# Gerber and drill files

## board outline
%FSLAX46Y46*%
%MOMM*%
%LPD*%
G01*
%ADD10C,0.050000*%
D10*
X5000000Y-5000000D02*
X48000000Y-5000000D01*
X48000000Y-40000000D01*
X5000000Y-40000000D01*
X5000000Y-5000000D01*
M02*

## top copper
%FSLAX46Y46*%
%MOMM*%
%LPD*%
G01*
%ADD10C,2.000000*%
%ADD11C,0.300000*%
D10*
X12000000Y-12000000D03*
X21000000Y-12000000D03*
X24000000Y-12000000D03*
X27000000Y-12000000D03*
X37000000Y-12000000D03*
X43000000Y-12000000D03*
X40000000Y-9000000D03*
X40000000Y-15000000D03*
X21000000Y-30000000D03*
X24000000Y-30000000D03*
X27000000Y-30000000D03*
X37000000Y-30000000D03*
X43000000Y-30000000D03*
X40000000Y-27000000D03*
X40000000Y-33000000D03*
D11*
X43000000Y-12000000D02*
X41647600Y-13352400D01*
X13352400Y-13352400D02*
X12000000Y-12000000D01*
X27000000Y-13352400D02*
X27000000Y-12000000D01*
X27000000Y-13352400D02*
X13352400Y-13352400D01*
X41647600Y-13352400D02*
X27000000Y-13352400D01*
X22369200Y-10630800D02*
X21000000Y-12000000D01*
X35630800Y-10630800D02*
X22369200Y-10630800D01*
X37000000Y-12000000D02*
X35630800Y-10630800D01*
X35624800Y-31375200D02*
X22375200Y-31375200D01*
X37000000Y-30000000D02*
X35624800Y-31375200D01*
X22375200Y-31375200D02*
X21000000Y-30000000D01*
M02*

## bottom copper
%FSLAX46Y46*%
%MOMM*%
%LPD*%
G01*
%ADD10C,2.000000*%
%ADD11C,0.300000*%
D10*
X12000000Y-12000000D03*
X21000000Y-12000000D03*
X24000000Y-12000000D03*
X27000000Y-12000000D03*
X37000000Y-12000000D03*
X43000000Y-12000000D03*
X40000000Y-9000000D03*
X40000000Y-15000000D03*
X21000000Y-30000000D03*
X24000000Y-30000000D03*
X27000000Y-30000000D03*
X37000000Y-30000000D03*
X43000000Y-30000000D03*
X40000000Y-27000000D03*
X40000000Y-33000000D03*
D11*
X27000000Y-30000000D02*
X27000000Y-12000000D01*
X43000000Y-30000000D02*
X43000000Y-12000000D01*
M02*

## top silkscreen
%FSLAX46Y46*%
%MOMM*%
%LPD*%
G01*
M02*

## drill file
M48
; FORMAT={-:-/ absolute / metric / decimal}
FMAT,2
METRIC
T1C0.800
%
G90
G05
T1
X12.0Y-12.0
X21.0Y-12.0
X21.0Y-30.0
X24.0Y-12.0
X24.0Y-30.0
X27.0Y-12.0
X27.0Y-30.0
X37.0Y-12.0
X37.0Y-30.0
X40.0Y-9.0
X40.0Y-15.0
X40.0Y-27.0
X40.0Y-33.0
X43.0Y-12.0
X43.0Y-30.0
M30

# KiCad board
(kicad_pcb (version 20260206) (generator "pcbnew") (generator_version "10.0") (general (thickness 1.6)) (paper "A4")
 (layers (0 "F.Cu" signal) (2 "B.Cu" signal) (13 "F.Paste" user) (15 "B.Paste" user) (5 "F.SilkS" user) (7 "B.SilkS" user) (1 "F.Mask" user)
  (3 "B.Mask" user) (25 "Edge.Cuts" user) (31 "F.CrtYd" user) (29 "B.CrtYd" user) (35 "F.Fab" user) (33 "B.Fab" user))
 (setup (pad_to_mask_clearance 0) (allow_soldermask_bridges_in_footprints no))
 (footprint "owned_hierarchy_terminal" (layer "F.Cu") (at 12 12)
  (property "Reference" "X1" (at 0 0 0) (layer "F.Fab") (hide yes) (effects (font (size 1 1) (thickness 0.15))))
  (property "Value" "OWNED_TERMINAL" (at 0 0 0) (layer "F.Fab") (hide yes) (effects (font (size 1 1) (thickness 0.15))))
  (pad "1" thru_hole circle (at 0 0) (size 2 2) (drill 0.8) (layers "*.Cu" "*.Mask") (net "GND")))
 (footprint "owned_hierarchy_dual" (layer "F.Cu") (at 24 12)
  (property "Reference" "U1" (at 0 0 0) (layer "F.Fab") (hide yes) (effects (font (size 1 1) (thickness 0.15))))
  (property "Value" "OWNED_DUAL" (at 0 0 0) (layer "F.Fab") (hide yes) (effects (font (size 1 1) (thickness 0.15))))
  (pad "1" thru_hole circle (at -3 0) (size 2 2) (drill 0.8) (layers "*.Cu" "*.Mask") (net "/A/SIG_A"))
  (pad "2" thru_hole circle (at 0 0) (size 2 2) (drill 0.8) (layers "*.Cu" "*.Mask") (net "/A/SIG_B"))
  (pad "3" thru_hole circle (at 3 0) (size 2 2) (drill 0.8) (layers "*.Cu" "*.Mask") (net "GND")))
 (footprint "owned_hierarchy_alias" (layer "F.Cu") (at 40 12)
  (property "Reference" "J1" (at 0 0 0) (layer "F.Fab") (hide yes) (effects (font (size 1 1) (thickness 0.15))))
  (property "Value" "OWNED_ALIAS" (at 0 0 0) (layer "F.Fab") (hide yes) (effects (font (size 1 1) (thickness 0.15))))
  (pad "R" thru_hole circle (at -3 0) (size 2 2) (drill 0.8) (layers "*.Cu" "*.Mask") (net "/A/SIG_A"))
  (pad "T" thru_hole circle (at 3 0) (size 2 2) (drill 0.8) (layers "*.Cu" "*.Mask") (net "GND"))
  (pad "MP" thru_hole circle (at 0 -3) (size 2 2) (drill 0.8) (layers "*.Cu" "*.Mask"))
  (pad "MP" thru_hole circle (at 0 3) (size 2 2) (drill 0.8) (layers "*.Cu" "*.Mask")))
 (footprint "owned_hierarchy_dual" (layer "F.Cu") (at 24 30)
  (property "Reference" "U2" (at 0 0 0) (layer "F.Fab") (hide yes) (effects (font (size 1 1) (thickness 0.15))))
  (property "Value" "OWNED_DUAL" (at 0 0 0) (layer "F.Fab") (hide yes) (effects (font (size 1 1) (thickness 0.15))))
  (pad "1" thru_hole circle (at -3 0) (size 2 2) (drill 0.8) (layers "*.Cu" "*.Mask") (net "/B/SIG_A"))
  (pad "2" thru_hole circle (at 0 0) (size 2 2) (drill 0.8) (layers "*.Cu" "*.Mask") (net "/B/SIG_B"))
  (pad "3" thru_hole circle (at 3 0) (size 2 2) (drill 0.8) (layers "*.Cu" "*.Mask") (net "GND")))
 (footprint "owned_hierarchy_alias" (layer "F.Cu") (at 40 30)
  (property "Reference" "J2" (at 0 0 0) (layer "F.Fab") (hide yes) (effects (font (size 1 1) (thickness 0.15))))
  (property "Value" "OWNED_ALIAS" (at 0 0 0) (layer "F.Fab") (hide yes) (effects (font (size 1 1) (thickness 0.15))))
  (pad "R" thru_hole circle (at -3 0) (size 2 2) (drill 0.8) (layers "*.Cu" "*.Mask") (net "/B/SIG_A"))
  (pad "T" thru_hole circle (at 3 0) (size 2 2) (drill 0.8) (layers "*.Cu" "*.Mask") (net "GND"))
  (pad "MP" thru_hole circle (at 0 -3) (size 2 2) (drill 0.8) (layers "*.Cu" "*.Mask"))
  (pad "MP" thru_hole circle (at 0 3) (size 2 2) (drill 0.8) (layers "*.Cu" "*.Mask")))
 (gr_rect (start 5 5) (end 48 40) (stroke (width 0.05) (type default)) (fill none) (layer "Edge.Cuts"))
 (segment (start 43 12) (end 41.6476 13.3524) (width 0.3) (layer "F.Cu") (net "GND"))
 (segment (start 13.3524 13.3524) (end 12 12) (width 0.3) (layer "F.Cu") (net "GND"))
 (segment (start 27 13.3524) (end 27 12) (width 0.3) (layer "F.Cu") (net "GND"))
 (segment (start 27 13.3524) (end 13.3524 13.3524) (width 0.3) (layer "F.Cu") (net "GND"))
 (segment (start 41.6476 13.3524) (end 27 13.3524) (width 0.3) (layer "F.Cu") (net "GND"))
 (segment (start 27 30) (end 27 12) (width 0.3) (layer "B.Cu") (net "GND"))
 (segment (start 43 30) (end 43 12) (width 0.3) (layer "B.Cu") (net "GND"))
 (segment (start 22.3692 10.6308) (end 21 12) (width 0.3) (layer "F.Cu") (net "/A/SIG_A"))
 (segment (start 35.6308 10.6308) (end 22.3692 10.6308) (width 0.3) (layer "F.Cu") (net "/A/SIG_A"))
 (segment (start 37 12) (end 35.6308 10.6308) (width 0.3) (layer "F.Cu") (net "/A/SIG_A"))
 (segment (start 35.6248 31.3752) (end 22.3752 31.3752) (width 0.3) (layer "F.Cu") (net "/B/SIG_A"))
 (segment (start 37 30) (end 35.6248 31.3752) (width 0.3) (layer "F.Cu") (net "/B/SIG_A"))
 (segment (start 22.3752 31.3752) (end 21 30) (width 0.3) (layer "F.Cu") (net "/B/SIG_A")))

